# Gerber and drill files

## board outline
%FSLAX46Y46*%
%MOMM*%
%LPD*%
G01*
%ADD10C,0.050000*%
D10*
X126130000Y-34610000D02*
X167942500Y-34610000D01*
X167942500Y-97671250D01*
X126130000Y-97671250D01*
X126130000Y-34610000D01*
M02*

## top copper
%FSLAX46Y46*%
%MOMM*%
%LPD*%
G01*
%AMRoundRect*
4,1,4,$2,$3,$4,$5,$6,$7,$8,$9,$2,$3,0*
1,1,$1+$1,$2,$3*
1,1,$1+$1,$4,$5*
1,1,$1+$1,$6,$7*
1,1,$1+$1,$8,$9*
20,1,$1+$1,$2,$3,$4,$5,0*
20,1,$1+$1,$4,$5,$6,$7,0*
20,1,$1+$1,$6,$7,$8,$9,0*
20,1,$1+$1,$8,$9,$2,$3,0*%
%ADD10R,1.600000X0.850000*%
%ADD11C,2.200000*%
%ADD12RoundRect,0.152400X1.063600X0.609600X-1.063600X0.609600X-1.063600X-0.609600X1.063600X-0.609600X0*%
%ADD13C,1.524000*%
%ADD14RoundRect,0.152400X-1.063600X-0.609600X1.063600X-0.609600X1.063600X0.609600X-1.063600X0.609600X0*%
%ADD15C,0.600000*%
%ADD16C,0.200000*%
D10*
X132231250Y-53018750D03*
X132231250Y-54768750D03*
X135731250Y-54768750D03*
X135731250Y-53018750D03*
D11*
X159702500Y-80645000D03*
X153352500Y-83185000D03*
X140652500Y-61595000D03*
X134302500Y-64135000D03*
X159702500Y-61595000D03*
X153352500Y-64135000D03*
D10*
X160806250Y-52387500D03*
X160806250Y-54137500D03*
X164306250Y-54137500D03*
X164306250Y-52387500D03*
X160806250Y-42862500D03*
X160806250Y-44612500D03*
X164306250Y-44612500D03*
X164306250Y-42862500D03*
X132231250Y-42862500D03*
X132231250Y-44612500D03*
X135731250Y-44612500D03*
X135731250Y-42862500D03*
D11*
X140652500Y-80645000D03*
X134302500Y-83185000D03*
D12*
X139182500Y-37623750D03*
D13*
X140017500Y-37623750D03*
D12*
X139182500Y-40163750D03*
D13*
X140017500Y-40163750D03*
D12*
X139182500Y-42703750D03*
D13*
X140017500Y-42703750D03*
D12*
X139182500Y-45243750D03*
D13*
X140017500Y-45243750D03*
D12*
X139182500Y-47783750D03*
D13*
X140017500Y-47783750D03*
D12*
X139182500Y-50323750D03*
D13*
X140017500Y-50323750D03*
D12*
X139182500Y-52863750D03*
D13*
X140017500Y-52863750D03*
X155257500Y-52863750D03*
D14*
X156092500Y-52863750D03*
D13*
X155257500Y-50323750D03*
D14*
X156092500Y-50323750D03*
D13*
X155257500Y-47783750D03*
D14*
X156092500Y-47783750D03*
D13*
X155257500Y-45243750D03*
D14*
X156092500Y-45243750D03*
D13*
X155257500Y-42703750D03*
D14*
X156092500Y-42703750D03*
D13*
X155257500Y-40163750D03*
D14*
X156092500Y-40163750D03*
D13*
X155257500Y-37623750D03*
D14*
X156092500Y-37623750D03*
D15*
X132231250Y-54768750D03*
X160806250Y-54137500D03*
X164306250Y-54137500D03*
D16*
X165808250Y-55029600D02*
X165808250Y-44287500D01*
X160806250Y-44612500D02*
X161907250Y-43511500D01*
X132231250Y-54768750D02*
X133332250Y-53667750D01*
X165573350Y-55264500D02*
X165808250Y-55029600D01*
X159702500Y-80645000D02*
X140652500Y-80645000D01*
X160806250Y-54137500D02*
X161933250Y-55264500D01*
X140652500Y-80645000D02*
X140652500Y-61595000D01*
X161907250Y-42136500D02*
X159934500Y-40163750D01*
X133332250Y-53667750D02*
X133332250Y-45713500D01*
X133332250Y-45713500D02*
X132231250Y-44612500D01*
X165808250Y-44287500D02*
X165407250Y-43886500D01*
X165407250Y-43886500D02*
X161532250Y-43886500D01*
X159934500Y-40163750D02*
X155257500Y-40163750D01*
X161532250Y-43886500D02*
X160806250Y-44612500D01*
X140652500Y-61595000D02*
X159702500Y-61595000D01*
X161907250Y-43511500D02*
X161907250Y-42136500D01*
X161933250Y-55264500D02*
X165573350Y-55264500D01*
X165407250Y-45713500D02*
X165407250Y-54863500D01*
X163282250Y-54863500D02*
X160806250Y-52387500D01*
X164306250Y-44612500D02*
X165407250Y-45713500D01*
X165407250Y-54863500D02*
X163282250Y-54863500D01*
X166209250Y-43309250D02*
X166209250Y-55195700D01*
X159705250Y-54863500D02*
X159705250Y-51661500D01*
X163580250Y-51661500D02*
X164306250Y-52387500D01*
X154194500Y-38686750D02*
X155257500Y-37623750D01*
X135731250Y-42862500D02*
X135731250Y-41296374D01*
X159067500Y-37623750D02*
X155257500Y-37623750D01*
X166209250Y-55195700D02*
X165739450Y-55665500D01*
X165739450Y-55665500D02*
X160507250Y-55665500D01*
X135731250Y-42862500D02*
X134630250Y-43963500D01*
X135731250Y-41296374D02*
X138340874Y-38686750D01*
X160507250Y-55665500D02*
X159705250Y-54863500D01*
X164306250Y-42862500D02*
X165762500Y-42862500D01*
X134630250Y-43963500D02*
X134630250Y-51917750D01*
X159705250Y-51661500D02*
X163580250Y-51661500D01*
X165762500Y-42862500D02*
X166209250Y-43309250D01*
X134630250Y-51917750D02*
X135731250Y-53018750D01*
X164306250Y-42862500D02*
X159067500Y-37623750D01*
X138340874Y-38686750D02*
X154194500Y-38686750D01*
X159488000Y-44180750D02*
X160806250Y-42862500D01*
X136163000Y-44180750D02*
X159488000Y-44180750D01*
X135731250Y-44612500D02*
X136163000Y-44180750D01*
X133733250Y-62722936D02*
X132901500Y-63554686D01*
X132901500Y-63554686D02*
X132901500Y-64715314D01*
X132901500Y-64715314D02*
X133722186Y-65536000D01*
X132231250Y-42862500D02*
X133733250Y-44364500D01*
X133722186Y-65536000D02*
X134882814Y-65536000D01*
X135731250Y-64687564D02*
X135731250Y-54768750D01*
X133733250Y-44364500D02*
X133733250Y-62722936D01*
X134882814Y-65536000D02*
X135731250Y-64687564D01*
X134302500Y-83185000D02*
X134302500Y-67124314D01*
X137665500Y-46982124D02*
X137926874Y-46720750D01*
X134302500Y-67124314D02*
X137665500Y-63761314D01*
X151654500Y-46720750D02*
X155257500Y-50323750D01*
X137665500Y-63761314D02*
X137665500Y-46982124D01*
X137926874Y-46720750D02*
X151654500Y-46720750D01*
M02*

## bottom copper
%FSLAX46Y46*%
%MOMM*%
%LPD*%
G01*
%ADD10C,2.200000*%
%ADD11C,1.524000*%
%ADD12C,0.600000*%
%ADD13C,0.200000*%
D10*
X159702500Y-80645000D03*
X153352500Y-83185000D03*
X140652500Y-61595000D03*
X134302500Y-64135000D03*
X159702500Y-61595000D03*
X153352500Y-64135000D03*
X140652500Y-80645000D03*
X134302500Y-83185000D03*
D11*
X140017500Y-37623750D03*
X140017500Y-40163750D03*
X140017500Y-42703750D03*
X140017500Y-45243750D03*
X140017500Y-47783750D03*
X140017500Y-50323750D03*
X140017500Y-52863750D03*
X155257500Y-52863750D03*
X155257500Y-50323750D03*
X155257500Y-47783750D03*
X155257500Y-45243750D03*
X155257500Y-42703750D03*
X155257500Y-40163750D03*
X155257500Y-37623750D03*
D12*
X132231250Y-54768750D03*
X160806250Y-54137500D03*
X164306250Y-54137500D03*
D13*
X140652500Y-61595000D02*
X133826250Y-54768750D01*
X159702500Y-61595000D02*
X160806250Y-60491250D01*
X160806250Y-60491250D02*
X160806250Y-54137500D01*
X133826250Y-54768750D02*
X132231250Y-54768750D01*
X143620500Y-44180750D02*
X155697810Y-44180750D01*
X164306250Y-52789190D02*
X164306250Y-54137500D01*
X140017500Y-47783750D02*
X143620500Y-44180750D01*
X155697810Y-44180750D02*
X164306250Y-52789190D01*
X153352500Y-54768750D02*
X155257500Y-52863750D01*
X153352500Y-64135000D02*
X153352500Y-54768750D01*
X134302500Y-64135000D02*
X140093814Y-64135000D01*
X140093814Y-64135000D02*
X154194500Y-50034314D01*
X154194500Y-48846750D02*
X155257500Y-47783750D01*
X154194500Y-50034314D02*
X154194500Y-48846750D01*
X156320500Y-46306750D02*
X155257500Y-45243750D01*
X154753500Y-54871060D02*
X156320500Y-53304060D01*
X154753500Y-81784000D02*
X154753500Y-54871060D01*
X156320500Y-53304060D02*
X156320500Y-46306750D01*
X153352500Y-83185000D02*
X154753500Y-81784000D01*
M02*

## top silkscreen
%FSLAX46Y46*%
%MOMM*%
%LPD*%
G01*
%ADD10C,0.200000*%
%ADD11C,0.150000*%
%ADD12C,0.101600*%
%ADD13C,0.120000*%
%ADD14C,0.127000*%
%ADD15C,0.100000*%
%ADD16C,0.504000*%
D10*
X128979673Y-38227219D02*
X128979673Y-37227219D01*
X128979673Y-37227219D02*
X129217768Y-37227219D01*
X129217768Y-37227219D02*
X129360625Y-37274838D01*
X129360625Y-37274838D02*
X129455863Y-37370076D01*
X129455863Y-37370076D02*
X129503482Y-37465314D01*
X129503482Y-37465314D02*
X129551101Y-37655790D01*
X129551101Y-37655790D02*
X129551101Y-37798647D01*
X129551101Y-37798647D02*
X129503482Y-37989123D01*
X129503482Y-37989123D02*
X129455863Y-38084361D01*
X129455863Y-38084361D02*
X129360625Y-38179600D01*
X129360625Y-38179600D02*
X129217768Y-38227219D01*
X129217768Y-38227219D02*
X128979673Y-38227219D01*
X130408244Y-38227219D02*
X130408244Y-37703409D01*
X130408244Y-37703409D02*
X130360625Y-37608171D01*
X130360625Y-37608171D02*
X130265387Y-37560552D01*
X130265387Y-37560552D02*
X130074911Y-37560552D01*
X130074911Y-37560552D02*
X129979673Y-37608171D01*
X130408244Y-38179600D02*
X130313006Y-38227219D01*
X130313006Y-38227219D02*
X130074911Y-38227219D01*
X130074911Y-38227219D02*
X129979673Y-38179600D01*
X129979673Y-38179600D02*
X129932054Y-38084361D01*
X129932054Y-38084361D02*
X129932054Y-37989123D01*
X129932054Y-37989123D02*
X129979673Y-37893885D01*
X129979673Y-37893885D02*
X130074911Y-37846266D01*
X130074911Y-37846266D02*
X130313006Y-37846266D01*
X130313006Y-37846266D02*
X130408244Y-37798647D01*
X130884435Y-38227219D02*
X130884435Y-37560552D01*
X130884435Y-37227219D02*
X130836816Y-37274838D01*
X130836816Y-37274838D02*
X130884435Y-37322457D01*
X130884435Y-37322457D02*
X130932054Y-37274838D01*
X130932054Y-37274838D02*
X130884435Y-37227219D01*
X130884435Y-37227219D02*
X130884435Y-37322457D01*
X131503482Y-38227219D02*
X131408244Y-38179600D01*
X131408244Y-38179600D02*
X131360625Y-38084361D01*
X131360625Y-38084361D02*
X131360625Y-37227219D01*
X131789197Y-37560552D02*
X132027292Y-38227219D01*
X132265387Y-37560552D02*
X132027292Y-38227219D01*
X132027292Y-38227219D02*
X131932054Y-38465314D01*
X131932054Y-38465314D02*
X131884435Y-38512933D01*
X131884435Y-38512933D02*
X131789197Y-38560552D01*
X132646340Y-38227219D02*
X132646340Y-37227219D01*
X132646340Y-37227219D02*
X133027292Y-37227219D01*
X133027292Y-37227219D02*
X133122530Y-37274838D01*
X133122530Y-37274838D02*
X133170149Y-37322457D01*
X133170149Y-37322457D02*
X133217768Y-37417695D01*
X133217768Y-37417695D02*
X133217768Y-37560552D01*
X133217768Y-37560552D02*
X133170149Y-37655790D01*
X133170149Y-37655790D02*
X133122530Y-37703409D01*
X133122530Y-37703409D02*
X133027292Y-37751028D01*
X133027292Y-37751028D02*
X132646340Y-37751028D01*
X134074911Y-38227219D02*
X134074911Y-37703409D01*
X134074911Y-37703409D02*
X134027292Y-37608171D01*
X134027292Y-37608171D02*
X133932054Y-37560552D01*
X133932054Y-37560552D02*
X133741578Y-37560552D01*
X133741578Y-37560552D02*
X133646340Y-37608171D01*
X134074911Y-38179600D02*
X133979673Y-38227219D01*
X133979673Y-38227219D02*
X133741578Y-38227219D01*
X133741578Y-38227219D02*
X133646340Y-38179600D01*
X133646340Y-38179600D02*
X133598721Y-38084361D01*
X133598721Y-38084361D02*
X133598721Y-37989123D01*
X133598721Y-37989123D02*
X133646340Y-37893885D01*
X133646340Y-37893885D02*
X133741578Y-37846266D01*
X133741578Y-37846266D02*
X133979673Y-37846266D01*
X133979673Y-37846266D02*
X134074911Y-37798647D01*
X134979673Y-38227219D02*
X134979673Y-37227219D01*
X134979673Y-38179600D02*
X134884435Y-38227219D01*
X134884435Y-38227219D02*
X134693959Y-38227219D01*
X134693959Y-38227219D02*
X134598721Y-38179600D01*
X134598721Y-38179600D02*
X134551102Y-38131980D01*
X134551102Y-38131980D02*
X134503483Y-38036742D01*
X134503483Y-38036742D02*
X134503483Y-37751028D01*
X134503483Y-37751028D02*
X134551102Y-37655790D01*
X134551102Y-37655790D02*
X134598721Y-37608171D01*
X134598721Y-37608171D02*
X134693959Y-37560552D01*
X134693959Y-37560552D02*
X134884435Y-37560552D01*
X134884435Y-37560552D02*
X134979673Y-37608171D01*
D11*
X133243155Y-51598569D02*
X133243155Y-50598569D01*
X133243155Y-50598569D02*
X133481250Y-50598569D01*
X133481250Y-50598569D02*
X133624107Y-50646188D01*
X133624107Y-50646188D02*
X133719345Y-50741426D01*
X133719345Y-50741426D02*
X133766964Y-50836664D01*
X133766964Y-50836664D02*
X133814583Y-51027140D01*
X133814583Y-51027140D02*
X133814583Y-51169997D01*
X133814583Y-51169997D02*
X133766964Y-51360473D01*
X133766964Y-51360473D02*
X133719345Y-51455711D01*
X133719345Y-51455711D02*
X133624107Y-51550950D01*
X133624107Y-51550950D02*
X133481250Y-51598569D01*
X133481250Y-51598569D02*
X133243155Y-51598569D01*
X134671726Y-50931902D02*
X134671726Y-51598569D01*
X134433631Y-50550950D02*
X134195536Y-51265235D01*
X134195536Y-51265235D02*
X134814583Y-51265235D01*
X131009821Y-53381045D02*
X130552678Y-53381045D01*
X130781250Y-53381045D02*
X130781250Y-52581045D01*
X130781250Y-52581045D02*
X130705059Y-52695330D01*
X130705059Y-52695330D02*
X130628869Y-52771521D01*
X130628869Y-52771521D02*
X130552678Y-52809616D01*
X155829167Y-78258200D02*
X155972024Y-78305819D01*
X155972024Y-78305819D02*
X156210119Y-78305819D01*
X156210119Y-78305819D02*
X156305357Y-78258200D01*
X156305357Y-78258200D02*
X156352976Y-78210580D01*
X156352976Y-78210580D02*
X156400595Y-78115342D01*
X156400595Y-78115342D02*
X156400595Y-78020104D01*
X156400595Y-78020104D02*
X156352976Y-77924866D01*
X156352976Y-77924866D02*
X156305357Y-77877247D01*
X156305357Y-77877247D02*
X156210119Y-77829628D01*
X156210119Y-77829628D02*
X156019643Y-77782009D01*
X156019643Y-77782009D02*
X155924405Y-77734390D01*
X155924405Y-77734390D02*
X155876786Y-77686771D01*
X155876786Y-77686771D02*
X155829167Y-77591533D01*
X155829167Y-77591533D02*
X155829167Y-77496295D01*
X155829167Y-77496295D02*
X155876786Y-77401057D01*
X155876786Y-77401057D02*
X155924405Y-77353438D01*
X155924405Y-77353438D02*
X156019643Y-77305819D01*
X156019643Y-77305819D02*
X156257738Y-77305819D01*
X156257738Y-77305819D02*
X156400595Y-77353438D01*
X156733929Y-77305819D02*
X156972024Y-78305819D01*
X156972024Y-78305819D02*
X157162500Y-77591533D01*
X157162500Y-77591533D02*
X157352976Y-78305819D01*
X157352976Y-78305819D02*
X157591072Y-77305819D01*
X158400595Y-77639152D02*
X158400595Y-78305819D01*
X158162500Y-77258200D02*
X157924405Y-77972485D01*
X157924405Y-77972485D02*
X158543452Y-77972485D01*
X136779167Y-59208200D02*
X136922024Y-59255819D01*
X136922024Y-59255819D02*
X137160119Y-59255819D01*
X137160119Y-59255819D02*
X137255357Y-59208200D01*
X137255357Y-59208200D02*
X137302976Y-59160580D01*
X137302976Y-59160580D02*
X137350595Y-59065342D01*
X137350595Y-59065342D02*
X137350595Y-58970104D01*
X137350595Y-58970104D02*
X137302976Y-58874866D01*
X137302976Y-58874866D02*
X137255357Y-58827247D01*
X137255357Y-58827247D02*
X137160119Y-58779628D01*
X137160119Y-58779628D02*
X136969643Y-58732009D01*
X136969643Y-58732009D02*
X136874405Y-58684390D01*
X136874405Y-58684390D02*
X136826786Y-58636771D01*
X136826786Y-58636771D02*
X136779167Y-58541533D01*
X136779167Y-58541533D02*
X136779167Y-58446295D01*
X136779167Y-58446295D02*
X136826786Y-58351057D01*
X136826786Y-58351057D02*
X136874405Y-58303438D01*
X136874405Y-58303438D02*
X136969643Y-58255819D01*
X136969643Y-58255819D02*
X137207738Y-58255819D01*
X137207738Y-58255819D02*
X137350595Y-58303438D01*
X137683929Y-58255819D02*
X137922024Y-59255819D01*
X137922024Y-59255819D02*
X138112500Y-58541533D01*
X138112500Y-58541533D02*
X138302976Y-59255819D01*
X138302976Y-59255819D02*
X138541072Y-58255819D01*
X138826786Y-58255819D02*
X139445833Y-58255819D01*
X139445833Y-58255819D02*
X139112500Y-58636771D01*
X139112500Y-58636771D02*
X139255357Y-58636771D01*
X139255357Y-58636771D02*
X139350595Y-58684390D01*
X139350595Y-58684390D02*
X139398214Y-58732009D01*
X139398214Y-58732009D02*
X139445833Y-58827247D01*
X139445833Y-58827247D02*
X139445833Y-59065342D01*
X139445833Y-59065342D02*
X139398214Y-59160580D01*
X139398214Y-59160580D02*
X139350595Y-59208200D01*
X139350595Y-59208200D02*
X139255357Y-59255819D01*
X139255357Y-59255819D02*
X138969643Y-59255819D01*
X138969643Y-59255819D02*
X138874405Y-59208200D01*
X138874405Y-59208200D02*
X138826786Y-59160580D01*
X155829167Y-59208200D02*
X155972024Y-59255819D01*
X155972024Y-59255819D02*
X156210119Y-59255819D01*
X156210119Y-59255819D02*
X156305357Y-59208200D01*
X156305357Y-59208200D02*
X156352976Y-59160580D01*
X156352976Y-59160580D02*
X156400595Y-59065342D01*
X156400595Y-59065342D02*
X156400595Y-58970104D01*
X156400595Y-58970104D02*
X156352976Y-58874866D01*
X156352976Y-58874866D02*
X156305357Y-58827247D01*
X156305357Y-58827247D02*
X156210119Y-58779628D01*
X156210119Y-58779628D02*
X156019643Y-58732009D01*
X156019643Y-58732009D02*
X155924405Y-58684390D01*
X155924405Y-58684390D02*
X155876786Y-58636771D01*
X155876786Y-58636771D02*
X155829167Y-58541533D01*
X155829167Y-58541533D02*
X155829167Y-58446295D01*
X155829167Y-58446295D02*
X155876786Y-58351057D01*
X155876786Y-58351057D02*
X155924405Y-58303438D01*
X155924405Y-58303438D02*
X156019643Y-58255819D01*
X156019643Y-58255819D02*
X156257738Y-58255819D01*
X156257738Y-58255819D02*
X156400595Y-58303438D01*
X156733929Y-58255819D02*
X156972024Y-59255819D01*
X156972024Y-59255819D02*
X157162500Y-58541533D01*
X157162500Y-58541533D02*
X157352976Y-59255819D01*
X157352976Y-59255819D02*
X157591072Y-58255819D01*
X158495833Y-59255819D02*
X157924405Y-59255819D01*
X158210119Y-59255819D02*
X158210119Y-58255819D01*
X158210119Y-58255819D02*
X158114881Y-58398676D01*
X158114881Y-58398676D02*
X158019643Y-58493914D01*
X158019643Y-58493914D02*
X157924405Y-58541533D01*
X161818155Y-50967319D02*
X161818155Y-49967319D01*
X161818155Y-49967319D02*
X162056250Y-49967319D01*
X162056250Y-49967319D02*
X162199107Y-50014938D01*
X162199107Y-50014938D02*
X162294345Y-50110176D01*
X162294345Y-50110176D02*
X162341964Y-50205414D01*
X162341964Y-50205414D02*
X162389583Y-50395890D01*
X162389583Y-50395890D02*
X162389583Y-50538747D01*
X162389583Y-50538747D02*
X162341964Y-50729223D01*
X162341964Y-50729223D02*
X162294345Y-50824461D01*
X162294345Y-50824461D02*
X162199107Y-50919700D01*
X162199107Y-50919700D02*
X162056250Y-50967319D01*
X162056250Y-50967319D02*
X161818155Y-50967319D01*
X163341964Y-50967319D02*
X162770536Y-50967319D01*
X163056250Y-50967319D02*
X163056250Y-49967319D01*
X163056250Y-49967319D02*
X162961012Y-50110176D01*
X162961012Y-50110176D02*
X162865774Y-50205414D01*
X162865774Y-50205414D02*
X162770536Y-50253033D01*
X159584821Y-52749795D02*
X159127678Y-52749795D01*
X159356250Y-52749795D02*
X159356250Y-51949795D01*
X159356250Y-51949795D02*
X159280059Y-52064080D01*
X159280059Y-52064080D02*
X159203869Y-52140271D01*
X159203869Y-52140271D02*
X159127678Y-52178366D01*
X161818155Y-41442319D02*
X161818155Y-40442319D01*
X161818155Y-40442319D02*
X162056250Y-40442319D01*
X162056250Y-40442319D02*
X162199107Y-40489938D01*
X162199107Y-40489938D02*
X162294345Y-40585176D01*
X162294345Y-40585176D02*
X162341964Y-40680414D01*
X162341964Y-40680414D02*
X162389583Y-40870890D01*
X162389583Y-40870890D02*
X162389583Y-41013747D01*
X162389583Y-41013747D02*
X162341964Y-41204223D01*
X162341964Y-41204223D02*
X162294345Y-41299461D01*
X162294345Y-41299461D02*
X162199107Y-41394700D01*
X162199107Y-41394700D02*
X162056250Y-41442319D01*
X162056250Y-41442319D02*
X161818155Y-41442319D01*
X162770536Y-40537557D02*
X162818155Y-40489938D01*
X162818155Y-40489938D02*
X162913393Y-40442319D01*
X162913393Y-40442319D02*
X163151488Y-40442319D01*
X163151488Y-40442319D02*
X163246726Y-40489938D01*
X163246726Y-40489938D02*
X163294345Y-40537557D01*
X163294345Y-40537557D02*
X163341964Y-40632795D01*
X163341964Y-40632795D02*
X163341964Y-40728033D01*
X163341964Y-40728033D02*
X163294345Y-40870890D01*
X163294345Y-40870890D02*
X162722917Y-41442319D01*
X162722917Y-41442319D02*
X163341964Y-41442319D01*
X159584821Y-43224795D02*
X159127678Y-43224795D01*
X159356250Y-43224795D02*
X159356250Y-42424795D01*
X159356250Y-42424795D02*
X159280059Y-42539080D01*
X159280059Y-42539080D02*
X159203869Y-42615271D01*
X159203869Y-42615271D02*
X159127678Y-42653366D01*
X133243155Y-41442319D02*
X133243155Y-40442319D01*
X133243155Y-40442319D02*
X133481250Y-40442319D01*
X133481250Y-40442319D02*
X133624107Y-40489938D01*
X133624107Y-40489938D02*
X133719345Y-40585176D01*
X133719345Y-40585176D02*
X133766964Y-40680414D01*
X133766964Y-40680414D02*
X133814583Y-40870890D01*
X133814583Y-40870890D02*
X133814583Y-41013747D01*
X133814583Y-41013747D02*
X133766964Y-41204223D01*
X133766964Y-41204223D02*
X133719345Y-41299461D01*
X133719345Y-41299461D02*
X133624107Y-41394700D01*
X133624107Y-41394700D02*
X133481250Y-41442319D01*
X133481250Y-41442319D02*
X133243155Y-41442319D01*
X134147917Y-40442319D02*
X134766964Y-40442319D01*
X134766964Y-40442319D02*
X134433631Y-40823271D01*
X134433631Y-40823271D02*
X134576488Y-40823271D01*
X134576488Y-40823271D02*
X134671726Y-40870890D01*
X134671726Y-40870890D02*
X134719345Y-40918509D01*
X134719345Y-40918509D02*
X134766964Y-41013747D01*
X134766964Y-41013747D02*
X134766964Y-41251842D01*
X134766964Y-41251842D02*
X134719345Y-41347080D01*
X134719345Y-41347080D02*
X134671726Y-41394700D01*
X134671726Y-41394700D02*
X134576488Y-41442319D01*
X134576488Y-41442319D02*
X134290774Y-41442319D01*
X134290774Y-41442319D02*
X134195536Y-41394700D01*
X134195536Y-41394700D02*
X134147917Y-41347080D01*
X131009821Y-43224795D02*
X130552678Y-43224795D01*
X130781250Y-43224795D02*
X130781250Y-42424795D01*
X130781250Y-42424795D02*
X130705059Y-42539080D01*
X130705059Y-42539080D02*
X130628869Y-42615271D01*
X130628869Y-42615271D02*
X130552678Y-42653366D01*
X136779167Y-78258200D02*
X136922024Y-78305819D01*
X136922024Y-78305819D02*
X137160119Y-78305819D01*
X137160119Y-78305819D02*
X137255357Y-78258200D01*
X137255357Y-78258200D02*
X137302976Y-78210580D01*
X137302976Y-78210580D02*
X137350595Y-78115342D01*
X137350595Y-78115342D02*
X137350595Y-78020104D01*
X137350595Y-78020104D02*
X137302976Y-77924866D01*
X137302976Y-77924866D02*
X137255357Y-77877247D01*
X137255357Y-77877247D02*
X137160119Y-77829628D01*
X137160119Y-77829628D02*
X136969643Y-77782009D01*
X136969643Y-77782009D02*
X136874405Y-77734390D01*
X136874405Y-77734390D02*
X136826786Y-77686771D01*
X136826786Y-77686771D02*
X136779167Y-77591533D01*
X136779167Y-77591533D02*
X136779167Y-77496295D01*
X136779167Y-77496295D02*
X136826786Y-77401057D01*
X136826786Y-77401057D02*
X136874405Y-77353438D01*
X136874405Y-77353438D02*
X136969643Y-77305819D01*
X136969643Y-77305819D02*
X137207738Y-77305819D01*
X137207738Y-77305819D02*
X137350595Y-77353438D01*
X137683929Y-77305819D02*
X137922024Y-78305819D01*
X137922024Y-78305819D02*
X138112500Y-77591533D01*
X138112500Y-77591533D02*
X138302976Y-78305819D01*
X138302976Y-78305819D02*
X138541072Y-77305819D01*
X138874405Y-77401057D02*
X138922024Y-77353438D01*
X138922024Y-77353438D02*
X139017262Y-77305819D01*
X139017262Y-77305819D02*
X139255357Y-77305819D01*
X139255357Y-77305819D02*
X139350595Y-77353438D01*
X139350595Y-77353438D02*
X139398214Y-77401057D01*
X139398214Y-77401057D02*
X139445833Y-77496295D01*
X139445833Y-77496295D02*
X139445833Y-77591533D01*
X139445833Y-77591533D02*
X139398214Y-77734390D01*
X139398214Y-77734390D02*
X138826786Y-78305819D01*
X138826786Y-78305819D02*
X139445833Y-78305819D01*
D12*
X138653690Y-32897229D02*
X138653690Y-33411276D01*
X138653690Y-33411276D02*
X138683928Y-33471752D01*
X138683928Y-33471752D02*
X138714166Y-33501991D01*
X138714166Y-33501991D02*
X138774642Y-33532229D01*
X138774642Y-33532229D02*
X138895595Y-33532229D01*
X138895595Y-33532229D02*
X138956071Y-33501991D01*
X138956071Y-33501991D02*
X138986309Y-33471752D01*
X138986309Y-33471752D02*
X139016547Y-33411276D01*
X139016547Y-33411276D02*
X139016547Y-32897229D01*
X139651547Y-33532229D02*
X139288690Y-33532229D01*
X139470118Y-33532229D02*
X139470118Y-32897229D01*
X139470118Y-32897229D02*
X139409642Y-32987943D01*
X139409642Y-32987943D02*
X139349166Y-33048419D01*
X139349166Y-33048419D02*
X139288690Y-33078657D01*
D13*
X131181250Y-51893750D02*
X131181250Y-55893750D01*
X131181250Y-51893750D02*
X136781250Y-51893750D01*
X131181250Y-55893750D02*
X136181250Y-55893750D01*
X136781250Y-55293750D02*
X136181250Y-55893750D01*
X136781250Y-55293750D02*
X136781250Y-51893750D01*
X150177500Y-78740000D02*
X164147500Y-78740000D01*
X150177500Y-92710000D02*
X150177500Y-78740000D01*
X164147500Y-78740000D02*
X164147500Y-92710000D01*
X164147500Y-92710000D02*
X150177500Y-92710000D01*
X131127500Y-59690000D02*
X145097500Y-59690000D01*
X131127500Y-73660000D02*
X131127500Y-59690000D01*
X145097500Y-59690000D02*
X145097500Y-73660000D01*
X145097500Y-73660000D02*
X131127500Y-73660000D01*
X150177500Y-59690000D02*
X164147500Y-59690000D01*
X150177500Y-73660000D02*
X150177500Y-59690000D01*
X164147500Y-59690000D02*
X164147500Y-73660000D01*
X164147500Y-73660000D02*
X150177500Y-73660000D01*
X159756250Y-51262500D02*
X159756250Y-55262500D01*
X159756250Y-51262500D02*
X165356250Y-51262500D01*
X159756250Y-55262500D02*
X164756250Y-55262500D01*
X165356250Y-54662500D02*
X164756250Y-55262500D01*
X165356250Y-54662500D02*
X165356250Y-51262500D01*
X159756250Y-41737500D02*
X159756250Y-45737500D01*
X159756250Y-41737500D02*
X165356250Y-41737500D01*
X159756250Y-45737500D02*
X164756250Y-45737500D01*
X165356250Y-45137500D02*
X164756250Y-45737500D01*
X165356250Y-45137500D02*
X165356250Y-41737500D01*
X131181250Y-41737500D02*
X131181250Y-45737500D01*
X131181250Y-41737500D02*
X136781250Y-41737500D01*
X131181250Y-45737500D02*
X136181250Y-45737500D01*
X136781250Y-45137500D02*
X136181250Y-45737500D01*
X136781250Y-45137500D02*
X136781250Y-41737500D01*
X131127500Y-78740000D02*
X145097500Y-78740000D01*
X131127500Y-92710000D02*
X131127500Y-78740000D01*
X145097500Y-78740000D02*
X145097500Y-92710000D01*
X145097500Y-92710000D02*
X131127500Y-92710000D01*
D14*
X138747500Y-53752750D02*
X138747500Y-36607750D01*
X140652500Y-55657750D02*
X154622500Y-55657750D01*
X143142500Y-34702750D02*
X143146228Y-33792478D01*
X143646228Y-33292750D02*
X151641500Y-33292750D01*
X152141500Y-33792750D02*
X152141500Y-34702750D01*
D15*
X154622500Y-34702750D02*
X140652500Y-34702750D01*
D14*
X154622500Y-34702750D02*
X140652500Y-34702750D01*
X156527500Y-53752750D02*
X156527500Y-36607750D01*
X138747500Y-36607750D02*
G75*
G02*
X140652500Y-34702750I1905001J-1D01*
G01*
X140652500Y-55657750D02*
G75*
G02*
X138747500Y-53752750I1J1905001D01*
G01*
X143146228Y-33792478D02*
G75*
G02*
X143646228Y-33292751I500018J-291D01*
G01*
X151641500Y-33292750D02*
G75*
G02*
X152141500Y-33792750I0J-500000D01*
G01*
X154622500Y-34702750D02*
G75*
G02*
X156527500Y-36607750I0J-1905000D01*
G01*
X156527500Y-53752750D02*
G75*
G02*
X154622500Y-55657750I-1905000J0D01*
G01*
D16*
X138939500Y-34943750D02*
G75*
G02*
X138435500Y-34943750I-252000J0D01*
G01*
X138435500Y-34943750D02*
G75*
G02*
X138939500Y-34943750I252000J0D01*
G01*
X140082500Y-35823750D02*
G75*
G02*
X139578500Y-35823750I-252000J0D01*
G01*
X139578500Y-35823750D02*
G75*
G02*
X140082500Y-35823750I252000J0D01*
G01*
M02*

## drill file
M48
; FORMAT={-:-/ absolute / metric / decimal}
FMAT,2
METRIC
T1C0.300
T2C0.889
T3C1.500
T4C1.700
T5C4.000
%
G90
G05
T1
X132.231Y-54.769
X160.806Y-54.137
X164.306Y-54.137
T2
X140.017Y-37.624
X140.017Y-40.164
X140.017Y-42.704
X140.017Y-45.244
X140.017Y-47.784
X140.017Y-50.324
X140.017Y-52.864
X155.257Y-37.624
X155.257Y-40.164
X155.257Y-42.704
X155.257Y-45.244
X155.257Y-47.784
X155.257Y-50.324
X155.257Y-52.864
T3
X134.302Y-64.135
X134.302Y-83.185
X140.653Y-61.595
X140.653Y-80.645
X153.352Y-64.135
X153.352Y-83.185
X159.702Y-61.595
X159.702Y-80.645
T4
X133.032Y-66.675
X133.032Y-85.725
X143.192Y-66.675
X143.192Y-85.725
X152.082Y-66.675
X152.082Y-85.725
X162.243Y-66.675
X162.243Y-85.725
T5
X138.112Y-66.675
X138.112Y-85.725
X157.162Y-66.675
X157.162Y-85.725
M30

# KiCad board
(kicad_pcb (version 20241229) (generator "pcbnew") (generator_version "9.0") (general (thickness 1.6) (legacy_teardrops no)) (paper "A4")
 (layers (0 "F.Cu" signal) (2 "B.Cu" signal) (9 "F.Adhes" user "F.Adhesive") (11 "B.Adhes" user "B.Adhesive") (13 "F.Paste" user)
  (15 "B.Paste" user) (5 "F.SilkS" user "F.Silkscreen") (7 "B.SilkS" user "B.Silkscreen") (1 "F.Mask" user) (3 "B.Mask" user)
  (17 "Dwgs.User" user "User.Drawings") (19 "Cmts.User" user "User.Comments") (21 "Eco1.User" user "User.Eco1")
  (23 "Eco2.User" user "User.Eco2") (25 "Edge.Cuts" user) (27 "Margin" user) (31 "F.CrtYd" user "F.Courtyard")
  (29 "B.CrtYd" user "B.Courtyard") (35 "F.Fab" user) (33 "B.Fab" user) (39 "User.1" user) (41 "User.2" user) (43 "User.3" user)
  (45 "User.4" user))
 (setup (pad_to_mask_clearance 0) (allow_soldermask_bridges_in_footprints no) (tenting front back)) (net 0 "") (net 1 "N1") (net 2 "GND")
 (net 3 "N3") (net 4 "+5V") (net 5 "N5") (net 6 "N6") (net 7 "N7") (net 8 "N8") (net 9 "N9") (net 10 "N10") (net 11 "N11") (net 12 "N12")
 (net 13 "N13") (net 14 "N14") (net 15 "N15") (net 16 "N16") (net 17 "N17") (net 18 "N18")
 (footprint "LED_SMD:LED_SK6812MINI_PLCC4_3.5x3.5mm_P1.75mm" (layer "F.Cu") (at 133.98125 53.89375)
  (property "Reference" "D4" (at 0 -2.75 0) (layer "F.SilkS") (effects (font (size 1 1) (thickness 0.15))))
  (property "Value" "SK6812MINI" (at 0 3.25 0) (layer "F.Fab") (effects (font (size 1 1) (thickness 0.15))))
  (fp_line (start -2.8 -2) (end -2.8 2) (stroke (width 0.12) (type default)) (layer "F.SilkS"))
  (fp_line (start -2.8 -2) (end 2.8 -2) (stroke (width 0.12) (type solid)) (layer "F.SilkS"))
  (fp_line (start -2.8 2) (end 2.2 2) (stroke (width 0.12) (type solid)) (layer "F.SilkS"))
  (fp_line (start 2.8 1.4) (end 2.2 2) (stroke (width 0.12) (type default)) (layer "F.SilkS"))
  (fp_line (start 2.8 1.4) (end 2.8 -2) (stroke (width 0.12) (type solid)) (layer "F.SilkS"))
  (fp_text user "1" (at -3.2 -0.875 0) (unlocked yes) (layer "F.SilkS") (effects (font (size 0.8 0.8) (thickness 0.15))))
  (pad "1" smd rect (at -1.75 -0.875) (size 1.6 0.85) (layers "F.Cu" "F.Mask" "F.Paste") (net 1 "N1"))
  (pad "2" smd rect (at -1.75 0.875) (size 1.6 0.85) (layers "F.Cu" "F.Mask" "F.Paste") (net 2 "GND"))
  (pad "3" smd rect (at 1.75 0.875) (size 1.6 0.85) (layers "F.Cu" "F.Mask" "F.Paste") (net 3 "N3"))
  (pad "4" smd rect (at 1.75 -0.875) (size 1.6 0.85) (layers "F.Cu" "F.Mask" "F.Paste") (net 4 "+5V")))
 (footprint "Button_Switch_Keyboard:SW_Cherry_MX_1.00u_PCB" (layer "F.Cu") (at 159.7025 80.645)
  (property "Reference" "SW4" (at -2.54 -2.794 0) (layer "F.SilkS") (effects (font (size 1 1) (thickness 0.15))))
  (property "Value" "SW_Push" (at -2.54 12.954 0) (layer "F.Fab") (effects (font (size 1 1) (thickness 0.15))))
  (fp_line (start -9.525 -1.905) (end 4.445 -1.905) (stroke (width 0.12) (type solid)) (layer "F.SilkS"))
  (fp_line (start -9.525 12.065) (end -9.525 -1.905) (stroke (width 0.12) (type solid)) (layer "F.SilkS"))
  (fp_line (start 4.445 -1.905) (end 4.445 12.065) (stroke (width 0.12) (type solid)) (layer "F.SilkS"))
  (fp_line (start 4.445 12.065) (end -9.525 12.065) (stroke (width 0.12) (type solid)) (layer "F.SilkS"))
  (pad "" np_thru_hole circle (at -7.62 5.08) (size 1.7 1.7) (drill 1.7) (layers "*.Cu" "*.Mask"))
  (pad "" np_thru_hole circle (at -2.54 5.08) (size 4 4) (drill 4) (layers "*.Cu" "*.Mask"))
  (pad "" np_thru_hole circle (at 2.54 5.08) (size 1.7 1.7) (drill 1.7) (layers "*.Cu" "*.Mask"))
  (pad "1" thru_hole circle (at 0 0) (size 2.2 2.2) (drill 1.5) (layers "*.Cu" "*.Mask") (remove_unused_layers no) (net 2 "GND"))
  (pad "2" thru_hole circle (at -6.35 2.54) (size 2.2 2.2) (drill 1.5) (layers "*.Cu" "*.Mask") (remove_unused_layers no) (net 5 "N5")))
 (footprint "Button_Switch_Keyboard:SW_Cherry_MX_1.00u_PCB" (layer "F.Cu") (at 140.6525 61.595)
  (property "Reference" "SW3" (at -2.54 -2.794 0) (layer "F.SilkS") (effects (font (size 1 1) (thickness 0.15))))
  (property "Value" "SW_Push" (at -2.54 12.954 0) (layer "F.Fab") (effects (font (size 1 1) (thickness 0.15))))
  (fp_line (start -9.525 -1.905) (end 4.445 -1.905) (stroke (width 0.12) (type solid)) (layer "F.SilkS"))
  (fp_line (start -9.525 12.065) (end -9.525 -1.905) (stroke (width 0.12) (type solid)) (layer "F.SilkS"))
  (fp_line (start 4.445 -1.905) (end 4.445 12.065) (stroke (width 0.12) (type solid)) (layer "F.SilkS"))
  (fp_line (start 4.445 12.065) (end -9.525 12.065) (stroke (width 0.12) (type solid)) (layer "F.SilkS"))
  (pad "" np_thru_hole circle (at -7.62 5.08) (size 1.7 1.7) (drill 1.7) (layers "*.Cu" "*.Mask"))
  (pad "" np_thru_hole circle (at -2.54 5.08) (size 4 4) (drill 4) (layers "*.Cu" "*.Mask"))
  (pad "" np_thru_hole circle (at 2.54 5.08) (size 1.7 1.7) (drill 1.7) (layers "*.Cu" "*.Mask"))
  (pad "1" thru_hole circle (at 0 0) (size 2.2 2.2) (drill 1.5) (layers "*.Cu" "*.Mask") (remove_unused_layers no) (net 2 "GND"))
  (pad "2" thru_hole circle (at -6.35 2.54) (size 2.2 2.2) (drill 1.5) (layers "*.Cu" "*.Mask") (remove_unused_layers no) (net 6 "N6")))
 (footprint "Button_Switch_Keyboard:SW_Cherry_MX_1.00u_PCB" (layer "F.Cu") (at 159.7025 61.595)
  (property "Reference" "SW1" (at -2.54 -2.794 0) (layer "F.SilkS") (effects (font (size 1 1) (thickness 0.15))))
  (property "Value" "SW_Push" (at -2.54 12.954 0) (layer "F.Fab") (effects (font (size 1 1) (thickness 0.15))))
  (fp_line (start -9.525 -1.905) (end 4.445 -1.905) (stroke (width 0.12) (type solid)) (layer "F.SilkS"))
  (fp_line (start -9.525 12.065) (end -9.525 -1.905) (stroke (width 0.12) (type solid)) (layer "F.SilkS"))
  (fp_line (start 4.445 -1.905) (end 4.445 12.065) (stroke (width 0.12) (type solid)) (layer "F.SilkS"))
  (fp_line (start 4.445 12.065) (end -9.525 12.065) (stroke (width 0.12) (type solid)) (layer "F.SilkS"))
  (pad "" np_thru_hole circle (at -7.62 5.08) (size 1.7 1.7) (drill 1.7) (layers "*.Cu" "*.Mask"))
  (pad "" np_thru_hole circle (at -2.54 5.08) (size 4 4) (drill 4) (layers "*.Cu" "*.Mask"))
  (pad "" np_thru_hole circle (at 2.54 5.08) (size 1.7 1.7) (drill 1.7) (layers "*.Cu" "*.Mask"))
  (pad "1" thru_hole circle (at 0 0) (size 2.2 2.2) (drill 1.5) (layers "*.Cu" "*.Mask") (remove_unused_layers no) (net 2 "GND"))
  (pad "2" thru_hole circle (at -6.35 2.54) (size 2.2 2.2) (drill 1.5) (layers "*.Cu" "*.Mask") (remove_unused_layers no) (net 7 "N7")))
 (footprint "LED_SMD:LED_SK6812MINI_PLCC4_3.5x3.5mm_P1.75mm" (layer "F.Cu") (at 162.55625 53.2625)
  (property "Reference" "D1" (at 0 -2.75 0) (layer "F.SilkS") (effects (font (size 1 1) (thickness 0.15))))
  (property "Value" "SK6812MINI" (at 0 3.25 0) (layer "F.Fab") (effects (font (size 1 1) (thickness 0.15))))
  (fp_line (start -2.8 -2) (end -2.8 2) (stroke (width 0.12) (type default)) (layer "F.SilkS"))
  (fp_line (start -2.8 -2) (end 2.8 -2) (stroke (width 0.12) (type solid)) (layer "F.SilkS"))
  (fp_line (start -2.8 2) (end 2.2 2) (stroke (width 0.12) (type solid)) (layer "F.SilkS"))
  (fp_line (start 2.8 1.4) (end 2.2 2) (stroke (width 0.12) (type default)) (layer "F.SilkS"))
  (fp_line (start 2.8 1.4) (end 2.8 -2) (stroke (width 0.12) (type solid)) (layer "F.SilkS"))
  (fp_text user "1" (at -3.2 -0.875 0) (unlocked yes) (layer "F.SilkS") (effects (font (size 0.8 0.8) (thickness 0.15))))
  (pad "1" smd rect (at -1.75 -0.875) (size 1.6 0.85) (layers "F.Cu" "F.Mask" "F.Paste") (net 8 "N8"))
  (pad "2" smd rect (at -1.75 0.875) (size 1.6 0.85) (layers "F.Cu" "F.Mask" "F.Paste") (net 2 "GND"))
  (pad "3" smd rect (at 1.75 0.875) (size 1.6 0.85) (layers "F.Cu" "F.Mask" "F.Paste") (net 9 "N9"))
  (pad "4" smd rect (at 1.75 -0.875) (size 1.6 0.85) (layers "F.Cu" "F.Mask" "F.Paste") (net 4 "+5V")))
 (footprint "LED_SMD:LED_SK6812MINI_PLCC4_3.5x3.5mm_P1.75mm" (layer "F.Cu") (at 162.55625 43.7375)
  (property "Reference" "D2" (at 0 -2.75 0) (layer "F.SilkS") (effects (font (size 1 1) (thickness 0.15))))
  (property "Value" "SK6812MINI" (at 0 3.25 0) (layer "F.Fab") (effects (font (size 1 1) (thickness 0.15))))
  (fp_line (start -2.8 -2) (end -2.8 2) (stroke (width 0.12) (type default)) (layer "F.SilkS"))
  (fp_line (start -2.8 -2) (end 2.8 -2) (stroke (width 0.12) (type solid)) (layer "F.SilkS"))
  (fp_line (start -2.8 2) (end 2.2 2) (stroke (width 0.12) (type solid)) (layer "F.SilkS"))
  (fp_line (start 2.8 1.4) (end 2.2 2) (stroke (width 0.12) (type default)) (layer "F.SilkS"))
  (fp_line (start 2.8 1.4) (end 2.8 -2) (stroke (width 0.12) (type solid)) (layer "F.SilkS"))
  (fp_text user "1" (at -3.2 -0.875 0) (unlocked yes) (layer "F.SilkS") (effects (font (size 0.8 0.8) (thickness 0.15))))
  (pad "1" smd rect (at -1.75 -0.875) (size 1.6 0.85) (layers "F.Cu" "F.Mask" "F.Paste") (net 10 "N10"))
  (pad "2" smd rect (at -1.75 0.875) (size 1.6 0.85) (layers "F.Cu" "F.Mask" "F.Paste") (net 2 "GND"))
  (pad "3" smd rect (at 1.75 0.875) (size 1.6 0.85) (layers "F.Cu" "F.Mask" "F.Paste") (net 8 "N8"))
  (pad "4" smd rect (at 1.75 -0.875) (size 1.6 0.85) (layers "F.Cu" "F.Mask" "F.Paste") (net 4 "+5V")))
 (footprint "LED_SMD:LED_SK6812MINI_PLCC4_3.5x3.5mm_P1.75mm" (layer "F.Cu") (at 133.98125 43.7375)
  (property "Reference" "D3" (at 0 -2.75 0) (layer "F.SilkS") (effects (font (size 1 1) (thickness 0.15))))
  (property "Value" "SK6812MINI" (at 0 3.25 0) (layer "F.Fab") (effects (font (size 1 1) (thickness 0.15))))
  (fp_line (start -2.8 -2) (end -2.8 2) (stroke (width 0.12) (type default)) (layer "F.SilkS"))
  (fp_line (start -2.8 -2) (end 2.8 -2) (stroke (width 0.12) (type solid)) (layer "F.SilkS"))
  (fp_line (start -2.8 2) (end 2.2 2) (stroke (width 0.12) (type solid)) (layer "F.SilkS"))
  (fp_line (start 2.8 1.4) (end 2.2 2) (stroke (width 0.12) (type default)) (layer "F.SilkS"))
  (fp_line (start 2.8 1.4) (end 2.8 -2) (stroke (width 0.12) (type solid)) (layer "F.SilkS"))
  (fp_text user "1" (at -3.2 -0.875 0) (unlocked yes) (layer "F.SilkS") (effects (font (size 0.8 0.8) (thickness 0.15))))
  (pad "1" smd rect (at -1.75 -0.875) (size 1.6 0.85) (layers "F.Cu" "F.Mask" "F.Paste") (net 3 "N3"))
  (pad "2" smd rect (at -1.75 0.875) (size 1.6 0.85) (layers "F.Cu" "F.Mask" "F.Paste") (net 2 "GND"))
  (pad "3" smd rect (at 1.75 0.875) (size 1.6 0.85) (layers "F.Cu" "F.Mask" "F.Paste") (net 10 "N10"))
  (pad "4" smd rect (at 1.75 -0.875) (size 1.6 0.85) (layers "F.Cu" "F.Mask" "F.Paste") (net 4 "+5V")))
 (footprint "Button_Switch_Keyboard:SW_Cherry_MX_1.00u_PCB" (layer "F.Cu") (at 140.6525 80.645)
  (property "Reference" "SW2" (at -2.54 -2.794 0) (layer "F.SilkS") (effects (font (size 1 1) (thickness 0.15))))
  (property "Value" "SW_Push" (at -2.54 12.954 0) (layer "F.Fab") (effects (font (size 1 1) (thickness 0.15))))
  (fp_line (start -9.525 -1.905) (end 4.445 -1.905) (stroke (width 0.12) (type solid)) (layer "F.SilkS"))
  (fp_line (start -9.525 12.065) (end -9.525 -1.905) (stroke (width 0.12) (type solid)) (layer "F.SilkS"))
  (fp_line (start 4.445 -1.905) (end 4.445 12.065) (stroke (width 0.12) (type solid)) (layer "F.SilkS"))
  (fp_line (start 4.445 12.065) (end -9.525 12.065) (stroke (width 0.12) (type solid)) (layer "F.SilkS"))
  (pad "" np_thru_hole circle (at -7.62 5.08) (size 1.7 1.7) (drill 1.7) (layers "*.Cu" "*.Mask"))
  (pad "" np_thru_hole circle (at -2.54 5.08) (size 4 4) (drill 4) (layers "*.Cu" "*.Mask"))
  (pad "" np_thru_hole circle (at 2.54 5.08) (size 1.7 1.7) (drill 1.7) (layers "*.Cu" "*.Mask"))
  (pad "1" thru_hole circle (at 0 0) (size 2.2 2.2) (drill 1.5) (layers "*.Cu" "*.Mask") (remove_unused_layers no) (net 2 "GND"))
  (pad "2" thru_hole circle (at -6.35 2.54) (size 2.2 2.2) (drill 1.5) (layers "*.Cu" "*.Mask") (remove_unused_layers no) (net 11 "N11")))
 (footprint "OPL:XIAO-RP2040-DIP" (layer "F.Cu") (at 147.6375 45.24375)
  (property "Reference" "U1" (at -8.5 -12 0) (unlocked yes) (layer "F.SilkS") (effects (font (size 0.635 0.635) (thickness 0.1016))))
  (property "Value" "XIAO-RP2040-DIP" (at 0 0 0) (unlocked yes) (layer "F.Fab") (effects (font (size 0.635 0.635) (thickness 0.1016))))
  (fp_line (start -8.89 8.509) (end -8.89 -8.636) (stroke (width 0.127) (type solid)) (layer "F.SilkS"))
  (fp_line (start -6.985 10.414) (end 6.985 10.414) (stroke (width 0.127) (type solid)) (layer "F.SilkS"))
  (fp_line (start -4.495 -10.541) (end -4.491272 -11.451272) (stroke (width 0.127) (type solid)) (layer "F.SilkS"))
  (fp_line (start -3.991272 -11.951) (end 4.004 -11.951) (stroke (width 0.127) (type solid)) (layer "F.SilkS"))
  (fp_line (start 4.504 -11.451) (end 4.504 -10.541) (stroke (width 0.127) (type solid)) (layer "F.SilkS"))
  (fp_line (start 6.985 -10.541) (end -6.985 -10.541) (stroke (width 0.1) (type solid)) (layer "F.SilkS"))
  (fp_line (start 6.985 -10.541) (end -6.985 -10.541) (stroke (width 0.127) (type solid)) (layer "F.SilkS"))
  (fp_line (start 8.89 8.509) (end 8.89 -8.636) (stroke (width 0.127) (type solid)) (layer "F.SilkS"))
  (fp_arc (start -8.89 -8.636) (mid -8.332038 -9.983038) (end -6.985 -10.541) (stroke (width 0.127) (type solid)) (layer "F.SilkS"))
  (fp_arc (start -6.985 10.414) (mid -8.332038 9.856038) (end -8.89 8.509) (stroke (width 0.127) (type solid)) (layer "F.SilkS"))
  (fp_arc (start -4.491272 -11.451272) (mid -4.344728 -11.80464) (end -3.991272 -11.951) (stroke (width 0.127) (type default))
   (layer "F.SilkS"))
  (fp_arc (start 4.004 -11.951) (mid 4.357553 -11.804553) (end 4.504 -11.451) (stroke (width 0.127) (type default)) (layer "F.SilkS"))
  (fp_arc (start 6.985 -10.541) (mid 8.332038 -9.983038) (end 8.89 -8.636) (stroke (width 0.127) (type solid)) (layer "F.SilkS"))
  (fp_arc (start 8.89 8.509) (mid 8.332038 9.856038) (end 6.985 10.414) (stroke (width 0.127) (type solid)) (layer "F.SilkS"))
  (fp_circle (center -8.95 -10.3) (end -8.95 -10.554) (stroke (width 0.5) (type solid)) (fill yes) (layer "F.SilkS"))
  (fp_circle (center -7.807 -9.42) (end -7.807 -9.674) (stroke (width 0.5) (type solid)) (fill yes) (layer "F.SilkS"))
  (pad "1" smd roundrect (at -8.455 -7.62 180) (size 2.432 1.524) (layers "F.Cu" "F.Mask") (roundrect_rratio 0.1) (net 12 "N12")
   (thermal_bridge_angle 45))
  (pad "1" thru_hole circle (at -7.62 -7.62 180) (size 1.524 1.524) (drill 0.889) (layers "*.Cu" "*.Mask") (remove_unused_layers no)
   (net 12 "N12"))
  (pad "2" smd roundrect (at -8.455 -5.08 180) (size 2.432 1.524) (layers "F.Cu" "F.Mask") (roundrect_rratio 0.1) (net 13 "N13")
   (thermal_bridge_angle 45))
  (pad "2" thru_hole circle (at -7.62 -5.08 180) (size 1.524 1.524) (drill 0.889) (layers "*.Cu" "*.Mask") (remove_unused_layers no)
   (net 13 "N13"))
  (pad "3" smd roundrect (at -8.455 -2.54 180) (size 2.432 1.524) (layers "F.Cu" "F.Mask") (roundrect_rratio 0.1) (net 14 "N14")
   (thermal_bridge_angle 45))
  (pad "3" thru_hole circle (at -7.62 -2.54 180) (size 1.524 1.524) (drill 0.889) (layers "*.Cu" "*.Mask") (remove_unused_layers no)
   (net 14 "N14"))
  (pad "4" smd roundrect (at -8.455 0 180) (size 2.432 1.524) (layers "F.Cu" "F.Mask") (roundrect_rratio 0.1) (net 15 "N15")
   (thermal_bridge_angle 45))
  (pad "4" thru_hole circle (at -7.62 0 180) (size 1.524 1.524) (drill 0.889) (layers "*.Cu" "*.Mask") (remove_unused_layers no)
   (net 15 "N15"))
  (pad "5" smd roundrect (at -8.455 2.54 180) (size 2.432 1.524) (layers "F.Cu" "F.Mask") (roundrect_rratio 0.1) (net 9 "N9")
   (thermal_bridge_angle 45))
  (pad "5" thru_hole circle (at -7.62 2.54 180) (size 1.524 1.524) (drill 0.889) (layers "*.Cu" "*.Mask") (remove_unused_layers no)
   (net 9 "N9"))
  (pad "6" smd roundrect (at -8.455 5.08 180) (size 2.432 1.524) (layers "F.Cu" "F.Mask") (roundrect_rratio 0.1) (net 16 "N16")
   (thermal_bridge_angle 45))
  (pad "6" thru_hole circle (at -7.62 5.08 180) (size 1.524 1.524) (drill 0.889) (layers "*.Cu" "*.Mask") (remove_unused_layers no)
   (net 16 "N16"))
  (pad "7" smd roundrect (at -8.455 7.62 180) (size 2.432 1.524) (layers "F.Cu" "F.Mask") (roundrect_rratio 0.1) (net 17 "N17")
   (thermal_bridge_angle 45))
  (pad "7" thru_hole circle (at -7.62 7.62 180) (size 1.524 1.524) (drill 0.889) (layers "*.Cu" "*.Mask") (remove_unused_layers no)
   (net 17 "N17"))
  (pad "8" thru_hole circle (at 7.62 7.62) (size 1.524 1.524) (drill 0.889) (layers "*.Cu" "*.Mask") (remove_unused_layers no) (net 7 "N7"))
  (pad "8" smd roundrect (at 8.455 7.62) (size 2.432 1.524) (layers "F.Cu" "F.Mask") (roundrect_rratio 0.1) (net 7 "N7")
   (thermal_bridge_angle 45))
  (pad "9" thru_hole circle (at 7.62 5.08) (size 1.524 1.524) (drill 0.889) (layers "*.Cu" "*.Mask") (remove_unused_layers no)
   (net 11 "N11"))
  (pad "9" smd roundrect (at 8.455 5.08) (size 2.432 1.524) (layers "F.Cu" "F.Mask") (roundrect_rratio 0.1) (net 11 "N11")
   (thermal_bridge_angle 45))
  (pad "10" thru_hole circle (at 7.62 2.54) (size 1.524 1.524) (drill 0.889) (layers "*.Cu" "*.Mask") (remove_unused_layers no) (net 6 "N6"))
  (pad "10" smd roundrect (at 8.455 2.54) (size 2.432 1.524) (layers "F.Cu" "F.Mask") (roundrect_rratio 0.1) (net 6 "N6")
   (thermal_bridge_angle 45))
  (pad "11" thru_hole circle (at 7.62 0) (size 1.524 1.524) (drill 0.889) (layers "*.Cu" "*.Mask") (remove_unused_layers no) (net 5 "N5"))
  (pad "11" smd roundrect (at 8.455 0) (size 2.432 1.524) (layers "F.Cu" "F.Mask") (roundrect_rratio 0.1) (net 5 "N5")
   (thermal_bridge_angle 45))
  (pad "12" thru_hole circle (at 7.62 -2.54) (size 1.524 1.524) (drill 0.889) (layers "*.Cu" "*.Mask") (remove_unused_layers no)
   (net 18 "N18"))
  (pad "12" smd roundrect (at 8.455 -2.54) (size 2.432 1.524) (layers "F.Cu" "F.Mask") (roundrect_rratio 0.1) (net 18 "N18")
   (thermal_bridge_angle 45))
  (pad "13" thru_hole circle (at 7.62 -5.08) (size 1.524 1.524) (drill 0.889) (layers "*.Cu" "*.Mask") (remove_unused_layers no)
   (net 2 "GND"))
  (pad "13" smd roundrect (at 8.455 -5.08) (size 2.432 1.524) (layers "F.Cu" "F.Mask") (roundrect_rratio 0.1) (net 2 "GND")
   (thermal_bridge_angle 45))
  (pad "14" thru_hole circle (at 7.62 -7.62) (size 1.524 1.524) (drill 0.889) (layers "*.Cu" "*.Mask") (remove_unused_layers no)
   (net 4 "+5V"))
  (pad "14" smd roundrect (at 8.455 -7.62) (size 2.432 1.524) (layers "F.Cu" "F.Mask") (roundrect_rratio 0.1) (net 4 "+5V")
   (thermal_bridge_angle 45)))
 (gr_rect (start 126.13 34.61) (end 167.9425 97.67125) (stroke (width 0.05) (type default)) (fill no) (layer "Edge.Cuts"))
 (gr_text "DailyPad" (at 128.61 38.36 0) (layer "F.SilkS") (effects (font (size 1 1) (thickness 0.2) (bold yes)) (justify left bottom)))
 (segment (start 165.80825 55.0296) (end 165.80825 44.2875) (width 0.2) (layer "F.Cu") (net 2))
 (segment (start 160.80625 44.6125) (end 161.90725 43.5115) (width 0.2) (layer "F.Cu") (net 2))
 (segment (start 132.23125 54.76875) (end 133.33225 53.66775) (width 0.2) (layer "F.Cu") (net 2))
 (segment (start 165.57335 55.2645) (end 165.80825 55.0296) (width 0.2) (layer "F.Cu") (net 2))
 (segment (start 159.7025 80.645) (end 140.6525 80.645) (width 0.2) (layer "F.Cu") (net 2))
 (segment (start 160.80625 54.1375) (end 161.93325 55.2645) (width 0.2) (layer "F.Cu") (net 2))
 (segment (start 140.6525 80.645) (end 140.6525 61.595) (width 0.2) (layer "F.Cu") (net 2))
 (segment (start 161.90725 42.1365) (end 159.9345 40.16375) (width 0.2) (layer "F.Cu") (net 2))
 (segment (start 133.33225 53.66775) (end 133.33225 45.7135) (width 0.2) (layer "F.Cu") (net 2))
 (segment (start 133.33225 45.7135) (end 132.23125 44.6125) (width 0.2) (layer "F.Cu") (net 2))
 (segment (start 165.80825 44.2875) (end 165.40725 43.8865) (width 0.2) (layer "F.Cu") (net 2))
 (segment (start 165.40725 43.8865) (end 161.53225 43.8865) (width 0.2) (layer "F.Cu") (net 2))
 (segment (start 159.9345 40.16375) (end 155.2575 40.16375) (width 0.2) (layer "F.Cu") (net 2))
 (segment (start 161.53225 43.8865) (end 160.80625 44.6125) (width 0.2) (layer "F.Cu") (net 2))
 (segment (start 140.6525 61.595) (end 159.7025 61.595) (width 0.2) (layer "F.Cu") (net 2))
 (segment (start 161.90725 43.5115) (end 161.90725 42.1365) (width 0.2) (layer "F.Cu") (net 2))
 (segment (start 161.93325 55.2645) (end 165.57335 55.2645) (width 0.2) (layer "F.Cu") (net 2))
 (via (at 132.23125 54.76875) (size 0.6) (drill 0.3) (layers "F.Cu" "B.Cu") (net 2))
 (via (at 160.80625 54.1375) (size 0.6) (drill 0.3) (layers "F.Cu" "B.Cu") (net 2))
 (segment (start 140.6525 61.595) (end 133.82625 54.76875) (width 0.2) (layer "B.Cu") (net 2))
 (segment (start 159.7025 61.595) (end 160.80625 60.49125) (width 0.2) (layer "B.Cu") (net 2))
 (segment (start 160.80625 60.49125) (end 160.80625 54.1375) (width 0.2) (layer "B.Cu") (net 2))
 (segment (start 133.82625 54.76875) (end 132.23125 54.76875) (width 0.2) (layer "B.Cu") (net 2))
 (segment (start 165.40725 45.7135) (end 165.40725 54.8635) (width 0.2) (layer "F.Cu") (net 8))
 (segment (start 163.28225 54.8635) (end 160.80625 52.3875) (width 0.2) (layer "F.Cu") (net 8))
 (segment (start 164.30625 44.6125) (end 165.40725 45.7135) (width 0.2) (layer "F.Cu") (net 8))
 (segment (start 165.40725 54.8635) (end 163.28225 54.8635) (width 0.2) (layer "F.Cu") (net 8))
 (segment (start 166.20925 43.30925) (end 166.20925 55.1957) (width 0.2) (layer "F.Cu") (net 4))
 (segment (start 159.70525 54.8635) (end 159.70525 51.6615) (width 0.2) (layer "F.Cu") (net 4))
 (segment (start 163.58025 51.6615) (end 164.30625 52.3875) (width 0.2) (layer "F.Cu") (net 4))
 (segment (start 154.1945 38.68675) (end 155.2575 37.62375) (width 0.2) (layer "F.Cu") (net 4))
 (segment (start 135.73125 42.8625) (end 135.73125 41.296374) (width 0.2) (layer "F.Cu") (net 4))
 (segment (start 159.0675 37.62375) (end 155.2575 37.62375) (width 0.2) (layer "F.Cu") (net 4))
 (segment (start 166.20925 55.1957) (end 165.73945 55.6655) (width 0.2) (layer "F.Cu") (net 4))
 (segment (start 165.73945 55.6655) (end 160.50725 55.6655) (width 0.2) (layer "F.Cu") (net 4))
 (segment (start 135.73125 42.8625) (end 134.63025 43.9635) (width 0.2) (layer "F.Cu") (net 4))
 (segment (start 135.73125 41.296374) (end 138.340874 38.68675) (width 0.2) (layer "F.Cu") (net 4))
 (segment (start 160.50725 55.6655) (end 159.70525 54.8635) (width 0.2) (layer "F.Cu") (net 4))
 (segment (start 164.30625 42.8625) (end 165.7625 42.8625) (width 0.2) (layer "F.Cu") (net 4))
 (segment (start 134.63025 43.9635) (end 134.63025 51.91775) (width 0.2) (layer "F.Cu") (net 4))
 (segment (start 159.70525 51.6615) (end 163.58025 51.6615) (width 0.2) (layer "F.Cu") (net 4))
 (segment (start 165.7625 42.8625) (end 166.20925 43.30925) (width 0.2) (layer "F.Cu") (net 4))
 (segment (start 134.63025 51.91775) (end 135.73125 53.01875) (width 0.2) (layer "F.Cu") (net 4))
 (segment (start 164.30625 42.8625) (end 159.0675 37.62375) (width 0.2) (layer "F.Cu") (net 4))
 (segment (start 138.340874 38.68675) (end 154.1945 38.68675) (width 0.2) (layer "F.Cu") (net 4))
 (via (at 164.30625 54.1375) (size 0.6) (drill 0.3) (layers "F.Cu" "B.Cu") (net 9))
 (segment (start 143.6205 44.18075) (end 155.69781 44.18075) (width 0.2) (layer "B.Cu") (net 9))
 (segment (start 164.30625 52.78919) (end 164.30625 54.1375) (width 0.2) (layer "B.Cu") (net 9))
 (segment (start 140.0175 47.78375) (end 143.6205 44.18075) (width 0.2) (layer "B.Cu") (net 9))
 (segment (start 155.69781 44.18075) (end 164.30625 52.78919) (width 0.2) (layer "B.Cu") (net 9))
 (segment (start 159.488 44.18075) (end 160.80625 42.8625) (width 0.2) (layer "F.Cu") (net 10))
 (segment (start 136.163 44.18075) (end 159.488 44.18075) (width 0.2) (layer "F.Cu") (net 10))
 (segment (start 135.73125 44.6125) (end 136.163 44.18075) (width 0.2) (layer "F.Cu") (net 10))
 (segment (start 133.73325 62.722936) (end 132.9015 63.554686) (width 0.2) (layer "F.Cu") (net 3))
 (segment (start 132.9015 63.554686) (end 132.9015 64.715314) (width 0.2) (layer "F.Cu") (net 3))
 (segment (start 132.9015 64.715314) (end 133.722186 65.536) (width 0.2) (layer "F.Cu") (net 3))
 (segment (start 132.23125 42.8625) (end 133.73325 44.3645) (width 0.2) (layer "F.Cu") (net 3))
 (segment (start 133.722186 65.536) (end 134.882814 65.536) (width 0.2) (layer "F.Cu") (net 3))
 (segment (start 135.73125 64.687564) (end 135.73125 54.76875) (width 0.2) (layer "F.Cu") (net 3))
 (segment (start 133.73325 44.3645) (end 133.73325 62.722936) (width 0.2) (layer "F.Cu") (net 3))
 (segment (start 134.882814 65.536) (end 135.73125 64.687564) (width 0.2) (layer "F.Cu") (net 3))
 (segment (start 153.3525 54.76875) (end 155.2575 52.86375) (width 0.2) (layer "B.Cu") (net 7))
 (segment (start 153.3525 64.135) (end 153.3525 54.76875) (width 0.2) (layer "B.Cu") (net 7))
 (segment (start 134.3025 83.185) (end 134.3025 67.124314) (width 0.2) (layer "F.Cu") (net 11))
 (segment (start 137.6655 46.982124) (end 137.926874 46.72075) (width 0.2) (layer "F.Cu") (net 11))
 (segment (start 134.3025 67.124314) (end 137.6655 63.761314) (width 0.2) (layer "F.Cu") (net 11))
 (segment (start 151.6545 46.72075) (end 155.2575 50.32375) (width 0.2) (layer "F.Cu") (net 11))
 (segment (start 137.6655 63.761314) (end 137.6655 46.982124) (width 0.2) (layer "F.Cu") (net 11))
 (segment (start 137.926874 46.72075) (end 151.6545 46.72075) (width 0.2) (layer "F.Cu") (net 11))
 (segment (start 134.3025 64.135) (end 140.093814 64.135) (width 0.2) (layer "B.Cu") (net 6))
 (segment (start 140.093814 64.135) (end 154.1945 50.034314) (width 0.2) (layer "B.Cu") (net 6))
 (segment (start 154.1945 48.84675) (end 155.2575 47.78375) (width 0.2) (layer "B.Cu") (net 6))
 (segment (start 154.1945 50.034314) (end 154.1945 48.84675) (width 0.2) (layer "B.Cu") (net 6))
 (segment (start 156.3205 46.30675) (end 155.2575 45.24375) (width 0.2) (layer "B.Cu") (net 5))
 (segment (start 154.7535 54.87106) (end 156.3205 53.30406) (width 0.2) (layer "B.Cu") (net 5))
 (segment (start 154.7535 81.784) (end 154.7535 54.87106) (width 0.2) (layer "B.Cu") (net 5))
 (segment (start 156.3205 53.30406) (end 156.3205 46.30675) (width 0.2) (layer "B.Cu") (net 5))
 (segment (start 153.3525 83.185) (end 154.7535 81.784) (width 0.2) (layer "B.Cu") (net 5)))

